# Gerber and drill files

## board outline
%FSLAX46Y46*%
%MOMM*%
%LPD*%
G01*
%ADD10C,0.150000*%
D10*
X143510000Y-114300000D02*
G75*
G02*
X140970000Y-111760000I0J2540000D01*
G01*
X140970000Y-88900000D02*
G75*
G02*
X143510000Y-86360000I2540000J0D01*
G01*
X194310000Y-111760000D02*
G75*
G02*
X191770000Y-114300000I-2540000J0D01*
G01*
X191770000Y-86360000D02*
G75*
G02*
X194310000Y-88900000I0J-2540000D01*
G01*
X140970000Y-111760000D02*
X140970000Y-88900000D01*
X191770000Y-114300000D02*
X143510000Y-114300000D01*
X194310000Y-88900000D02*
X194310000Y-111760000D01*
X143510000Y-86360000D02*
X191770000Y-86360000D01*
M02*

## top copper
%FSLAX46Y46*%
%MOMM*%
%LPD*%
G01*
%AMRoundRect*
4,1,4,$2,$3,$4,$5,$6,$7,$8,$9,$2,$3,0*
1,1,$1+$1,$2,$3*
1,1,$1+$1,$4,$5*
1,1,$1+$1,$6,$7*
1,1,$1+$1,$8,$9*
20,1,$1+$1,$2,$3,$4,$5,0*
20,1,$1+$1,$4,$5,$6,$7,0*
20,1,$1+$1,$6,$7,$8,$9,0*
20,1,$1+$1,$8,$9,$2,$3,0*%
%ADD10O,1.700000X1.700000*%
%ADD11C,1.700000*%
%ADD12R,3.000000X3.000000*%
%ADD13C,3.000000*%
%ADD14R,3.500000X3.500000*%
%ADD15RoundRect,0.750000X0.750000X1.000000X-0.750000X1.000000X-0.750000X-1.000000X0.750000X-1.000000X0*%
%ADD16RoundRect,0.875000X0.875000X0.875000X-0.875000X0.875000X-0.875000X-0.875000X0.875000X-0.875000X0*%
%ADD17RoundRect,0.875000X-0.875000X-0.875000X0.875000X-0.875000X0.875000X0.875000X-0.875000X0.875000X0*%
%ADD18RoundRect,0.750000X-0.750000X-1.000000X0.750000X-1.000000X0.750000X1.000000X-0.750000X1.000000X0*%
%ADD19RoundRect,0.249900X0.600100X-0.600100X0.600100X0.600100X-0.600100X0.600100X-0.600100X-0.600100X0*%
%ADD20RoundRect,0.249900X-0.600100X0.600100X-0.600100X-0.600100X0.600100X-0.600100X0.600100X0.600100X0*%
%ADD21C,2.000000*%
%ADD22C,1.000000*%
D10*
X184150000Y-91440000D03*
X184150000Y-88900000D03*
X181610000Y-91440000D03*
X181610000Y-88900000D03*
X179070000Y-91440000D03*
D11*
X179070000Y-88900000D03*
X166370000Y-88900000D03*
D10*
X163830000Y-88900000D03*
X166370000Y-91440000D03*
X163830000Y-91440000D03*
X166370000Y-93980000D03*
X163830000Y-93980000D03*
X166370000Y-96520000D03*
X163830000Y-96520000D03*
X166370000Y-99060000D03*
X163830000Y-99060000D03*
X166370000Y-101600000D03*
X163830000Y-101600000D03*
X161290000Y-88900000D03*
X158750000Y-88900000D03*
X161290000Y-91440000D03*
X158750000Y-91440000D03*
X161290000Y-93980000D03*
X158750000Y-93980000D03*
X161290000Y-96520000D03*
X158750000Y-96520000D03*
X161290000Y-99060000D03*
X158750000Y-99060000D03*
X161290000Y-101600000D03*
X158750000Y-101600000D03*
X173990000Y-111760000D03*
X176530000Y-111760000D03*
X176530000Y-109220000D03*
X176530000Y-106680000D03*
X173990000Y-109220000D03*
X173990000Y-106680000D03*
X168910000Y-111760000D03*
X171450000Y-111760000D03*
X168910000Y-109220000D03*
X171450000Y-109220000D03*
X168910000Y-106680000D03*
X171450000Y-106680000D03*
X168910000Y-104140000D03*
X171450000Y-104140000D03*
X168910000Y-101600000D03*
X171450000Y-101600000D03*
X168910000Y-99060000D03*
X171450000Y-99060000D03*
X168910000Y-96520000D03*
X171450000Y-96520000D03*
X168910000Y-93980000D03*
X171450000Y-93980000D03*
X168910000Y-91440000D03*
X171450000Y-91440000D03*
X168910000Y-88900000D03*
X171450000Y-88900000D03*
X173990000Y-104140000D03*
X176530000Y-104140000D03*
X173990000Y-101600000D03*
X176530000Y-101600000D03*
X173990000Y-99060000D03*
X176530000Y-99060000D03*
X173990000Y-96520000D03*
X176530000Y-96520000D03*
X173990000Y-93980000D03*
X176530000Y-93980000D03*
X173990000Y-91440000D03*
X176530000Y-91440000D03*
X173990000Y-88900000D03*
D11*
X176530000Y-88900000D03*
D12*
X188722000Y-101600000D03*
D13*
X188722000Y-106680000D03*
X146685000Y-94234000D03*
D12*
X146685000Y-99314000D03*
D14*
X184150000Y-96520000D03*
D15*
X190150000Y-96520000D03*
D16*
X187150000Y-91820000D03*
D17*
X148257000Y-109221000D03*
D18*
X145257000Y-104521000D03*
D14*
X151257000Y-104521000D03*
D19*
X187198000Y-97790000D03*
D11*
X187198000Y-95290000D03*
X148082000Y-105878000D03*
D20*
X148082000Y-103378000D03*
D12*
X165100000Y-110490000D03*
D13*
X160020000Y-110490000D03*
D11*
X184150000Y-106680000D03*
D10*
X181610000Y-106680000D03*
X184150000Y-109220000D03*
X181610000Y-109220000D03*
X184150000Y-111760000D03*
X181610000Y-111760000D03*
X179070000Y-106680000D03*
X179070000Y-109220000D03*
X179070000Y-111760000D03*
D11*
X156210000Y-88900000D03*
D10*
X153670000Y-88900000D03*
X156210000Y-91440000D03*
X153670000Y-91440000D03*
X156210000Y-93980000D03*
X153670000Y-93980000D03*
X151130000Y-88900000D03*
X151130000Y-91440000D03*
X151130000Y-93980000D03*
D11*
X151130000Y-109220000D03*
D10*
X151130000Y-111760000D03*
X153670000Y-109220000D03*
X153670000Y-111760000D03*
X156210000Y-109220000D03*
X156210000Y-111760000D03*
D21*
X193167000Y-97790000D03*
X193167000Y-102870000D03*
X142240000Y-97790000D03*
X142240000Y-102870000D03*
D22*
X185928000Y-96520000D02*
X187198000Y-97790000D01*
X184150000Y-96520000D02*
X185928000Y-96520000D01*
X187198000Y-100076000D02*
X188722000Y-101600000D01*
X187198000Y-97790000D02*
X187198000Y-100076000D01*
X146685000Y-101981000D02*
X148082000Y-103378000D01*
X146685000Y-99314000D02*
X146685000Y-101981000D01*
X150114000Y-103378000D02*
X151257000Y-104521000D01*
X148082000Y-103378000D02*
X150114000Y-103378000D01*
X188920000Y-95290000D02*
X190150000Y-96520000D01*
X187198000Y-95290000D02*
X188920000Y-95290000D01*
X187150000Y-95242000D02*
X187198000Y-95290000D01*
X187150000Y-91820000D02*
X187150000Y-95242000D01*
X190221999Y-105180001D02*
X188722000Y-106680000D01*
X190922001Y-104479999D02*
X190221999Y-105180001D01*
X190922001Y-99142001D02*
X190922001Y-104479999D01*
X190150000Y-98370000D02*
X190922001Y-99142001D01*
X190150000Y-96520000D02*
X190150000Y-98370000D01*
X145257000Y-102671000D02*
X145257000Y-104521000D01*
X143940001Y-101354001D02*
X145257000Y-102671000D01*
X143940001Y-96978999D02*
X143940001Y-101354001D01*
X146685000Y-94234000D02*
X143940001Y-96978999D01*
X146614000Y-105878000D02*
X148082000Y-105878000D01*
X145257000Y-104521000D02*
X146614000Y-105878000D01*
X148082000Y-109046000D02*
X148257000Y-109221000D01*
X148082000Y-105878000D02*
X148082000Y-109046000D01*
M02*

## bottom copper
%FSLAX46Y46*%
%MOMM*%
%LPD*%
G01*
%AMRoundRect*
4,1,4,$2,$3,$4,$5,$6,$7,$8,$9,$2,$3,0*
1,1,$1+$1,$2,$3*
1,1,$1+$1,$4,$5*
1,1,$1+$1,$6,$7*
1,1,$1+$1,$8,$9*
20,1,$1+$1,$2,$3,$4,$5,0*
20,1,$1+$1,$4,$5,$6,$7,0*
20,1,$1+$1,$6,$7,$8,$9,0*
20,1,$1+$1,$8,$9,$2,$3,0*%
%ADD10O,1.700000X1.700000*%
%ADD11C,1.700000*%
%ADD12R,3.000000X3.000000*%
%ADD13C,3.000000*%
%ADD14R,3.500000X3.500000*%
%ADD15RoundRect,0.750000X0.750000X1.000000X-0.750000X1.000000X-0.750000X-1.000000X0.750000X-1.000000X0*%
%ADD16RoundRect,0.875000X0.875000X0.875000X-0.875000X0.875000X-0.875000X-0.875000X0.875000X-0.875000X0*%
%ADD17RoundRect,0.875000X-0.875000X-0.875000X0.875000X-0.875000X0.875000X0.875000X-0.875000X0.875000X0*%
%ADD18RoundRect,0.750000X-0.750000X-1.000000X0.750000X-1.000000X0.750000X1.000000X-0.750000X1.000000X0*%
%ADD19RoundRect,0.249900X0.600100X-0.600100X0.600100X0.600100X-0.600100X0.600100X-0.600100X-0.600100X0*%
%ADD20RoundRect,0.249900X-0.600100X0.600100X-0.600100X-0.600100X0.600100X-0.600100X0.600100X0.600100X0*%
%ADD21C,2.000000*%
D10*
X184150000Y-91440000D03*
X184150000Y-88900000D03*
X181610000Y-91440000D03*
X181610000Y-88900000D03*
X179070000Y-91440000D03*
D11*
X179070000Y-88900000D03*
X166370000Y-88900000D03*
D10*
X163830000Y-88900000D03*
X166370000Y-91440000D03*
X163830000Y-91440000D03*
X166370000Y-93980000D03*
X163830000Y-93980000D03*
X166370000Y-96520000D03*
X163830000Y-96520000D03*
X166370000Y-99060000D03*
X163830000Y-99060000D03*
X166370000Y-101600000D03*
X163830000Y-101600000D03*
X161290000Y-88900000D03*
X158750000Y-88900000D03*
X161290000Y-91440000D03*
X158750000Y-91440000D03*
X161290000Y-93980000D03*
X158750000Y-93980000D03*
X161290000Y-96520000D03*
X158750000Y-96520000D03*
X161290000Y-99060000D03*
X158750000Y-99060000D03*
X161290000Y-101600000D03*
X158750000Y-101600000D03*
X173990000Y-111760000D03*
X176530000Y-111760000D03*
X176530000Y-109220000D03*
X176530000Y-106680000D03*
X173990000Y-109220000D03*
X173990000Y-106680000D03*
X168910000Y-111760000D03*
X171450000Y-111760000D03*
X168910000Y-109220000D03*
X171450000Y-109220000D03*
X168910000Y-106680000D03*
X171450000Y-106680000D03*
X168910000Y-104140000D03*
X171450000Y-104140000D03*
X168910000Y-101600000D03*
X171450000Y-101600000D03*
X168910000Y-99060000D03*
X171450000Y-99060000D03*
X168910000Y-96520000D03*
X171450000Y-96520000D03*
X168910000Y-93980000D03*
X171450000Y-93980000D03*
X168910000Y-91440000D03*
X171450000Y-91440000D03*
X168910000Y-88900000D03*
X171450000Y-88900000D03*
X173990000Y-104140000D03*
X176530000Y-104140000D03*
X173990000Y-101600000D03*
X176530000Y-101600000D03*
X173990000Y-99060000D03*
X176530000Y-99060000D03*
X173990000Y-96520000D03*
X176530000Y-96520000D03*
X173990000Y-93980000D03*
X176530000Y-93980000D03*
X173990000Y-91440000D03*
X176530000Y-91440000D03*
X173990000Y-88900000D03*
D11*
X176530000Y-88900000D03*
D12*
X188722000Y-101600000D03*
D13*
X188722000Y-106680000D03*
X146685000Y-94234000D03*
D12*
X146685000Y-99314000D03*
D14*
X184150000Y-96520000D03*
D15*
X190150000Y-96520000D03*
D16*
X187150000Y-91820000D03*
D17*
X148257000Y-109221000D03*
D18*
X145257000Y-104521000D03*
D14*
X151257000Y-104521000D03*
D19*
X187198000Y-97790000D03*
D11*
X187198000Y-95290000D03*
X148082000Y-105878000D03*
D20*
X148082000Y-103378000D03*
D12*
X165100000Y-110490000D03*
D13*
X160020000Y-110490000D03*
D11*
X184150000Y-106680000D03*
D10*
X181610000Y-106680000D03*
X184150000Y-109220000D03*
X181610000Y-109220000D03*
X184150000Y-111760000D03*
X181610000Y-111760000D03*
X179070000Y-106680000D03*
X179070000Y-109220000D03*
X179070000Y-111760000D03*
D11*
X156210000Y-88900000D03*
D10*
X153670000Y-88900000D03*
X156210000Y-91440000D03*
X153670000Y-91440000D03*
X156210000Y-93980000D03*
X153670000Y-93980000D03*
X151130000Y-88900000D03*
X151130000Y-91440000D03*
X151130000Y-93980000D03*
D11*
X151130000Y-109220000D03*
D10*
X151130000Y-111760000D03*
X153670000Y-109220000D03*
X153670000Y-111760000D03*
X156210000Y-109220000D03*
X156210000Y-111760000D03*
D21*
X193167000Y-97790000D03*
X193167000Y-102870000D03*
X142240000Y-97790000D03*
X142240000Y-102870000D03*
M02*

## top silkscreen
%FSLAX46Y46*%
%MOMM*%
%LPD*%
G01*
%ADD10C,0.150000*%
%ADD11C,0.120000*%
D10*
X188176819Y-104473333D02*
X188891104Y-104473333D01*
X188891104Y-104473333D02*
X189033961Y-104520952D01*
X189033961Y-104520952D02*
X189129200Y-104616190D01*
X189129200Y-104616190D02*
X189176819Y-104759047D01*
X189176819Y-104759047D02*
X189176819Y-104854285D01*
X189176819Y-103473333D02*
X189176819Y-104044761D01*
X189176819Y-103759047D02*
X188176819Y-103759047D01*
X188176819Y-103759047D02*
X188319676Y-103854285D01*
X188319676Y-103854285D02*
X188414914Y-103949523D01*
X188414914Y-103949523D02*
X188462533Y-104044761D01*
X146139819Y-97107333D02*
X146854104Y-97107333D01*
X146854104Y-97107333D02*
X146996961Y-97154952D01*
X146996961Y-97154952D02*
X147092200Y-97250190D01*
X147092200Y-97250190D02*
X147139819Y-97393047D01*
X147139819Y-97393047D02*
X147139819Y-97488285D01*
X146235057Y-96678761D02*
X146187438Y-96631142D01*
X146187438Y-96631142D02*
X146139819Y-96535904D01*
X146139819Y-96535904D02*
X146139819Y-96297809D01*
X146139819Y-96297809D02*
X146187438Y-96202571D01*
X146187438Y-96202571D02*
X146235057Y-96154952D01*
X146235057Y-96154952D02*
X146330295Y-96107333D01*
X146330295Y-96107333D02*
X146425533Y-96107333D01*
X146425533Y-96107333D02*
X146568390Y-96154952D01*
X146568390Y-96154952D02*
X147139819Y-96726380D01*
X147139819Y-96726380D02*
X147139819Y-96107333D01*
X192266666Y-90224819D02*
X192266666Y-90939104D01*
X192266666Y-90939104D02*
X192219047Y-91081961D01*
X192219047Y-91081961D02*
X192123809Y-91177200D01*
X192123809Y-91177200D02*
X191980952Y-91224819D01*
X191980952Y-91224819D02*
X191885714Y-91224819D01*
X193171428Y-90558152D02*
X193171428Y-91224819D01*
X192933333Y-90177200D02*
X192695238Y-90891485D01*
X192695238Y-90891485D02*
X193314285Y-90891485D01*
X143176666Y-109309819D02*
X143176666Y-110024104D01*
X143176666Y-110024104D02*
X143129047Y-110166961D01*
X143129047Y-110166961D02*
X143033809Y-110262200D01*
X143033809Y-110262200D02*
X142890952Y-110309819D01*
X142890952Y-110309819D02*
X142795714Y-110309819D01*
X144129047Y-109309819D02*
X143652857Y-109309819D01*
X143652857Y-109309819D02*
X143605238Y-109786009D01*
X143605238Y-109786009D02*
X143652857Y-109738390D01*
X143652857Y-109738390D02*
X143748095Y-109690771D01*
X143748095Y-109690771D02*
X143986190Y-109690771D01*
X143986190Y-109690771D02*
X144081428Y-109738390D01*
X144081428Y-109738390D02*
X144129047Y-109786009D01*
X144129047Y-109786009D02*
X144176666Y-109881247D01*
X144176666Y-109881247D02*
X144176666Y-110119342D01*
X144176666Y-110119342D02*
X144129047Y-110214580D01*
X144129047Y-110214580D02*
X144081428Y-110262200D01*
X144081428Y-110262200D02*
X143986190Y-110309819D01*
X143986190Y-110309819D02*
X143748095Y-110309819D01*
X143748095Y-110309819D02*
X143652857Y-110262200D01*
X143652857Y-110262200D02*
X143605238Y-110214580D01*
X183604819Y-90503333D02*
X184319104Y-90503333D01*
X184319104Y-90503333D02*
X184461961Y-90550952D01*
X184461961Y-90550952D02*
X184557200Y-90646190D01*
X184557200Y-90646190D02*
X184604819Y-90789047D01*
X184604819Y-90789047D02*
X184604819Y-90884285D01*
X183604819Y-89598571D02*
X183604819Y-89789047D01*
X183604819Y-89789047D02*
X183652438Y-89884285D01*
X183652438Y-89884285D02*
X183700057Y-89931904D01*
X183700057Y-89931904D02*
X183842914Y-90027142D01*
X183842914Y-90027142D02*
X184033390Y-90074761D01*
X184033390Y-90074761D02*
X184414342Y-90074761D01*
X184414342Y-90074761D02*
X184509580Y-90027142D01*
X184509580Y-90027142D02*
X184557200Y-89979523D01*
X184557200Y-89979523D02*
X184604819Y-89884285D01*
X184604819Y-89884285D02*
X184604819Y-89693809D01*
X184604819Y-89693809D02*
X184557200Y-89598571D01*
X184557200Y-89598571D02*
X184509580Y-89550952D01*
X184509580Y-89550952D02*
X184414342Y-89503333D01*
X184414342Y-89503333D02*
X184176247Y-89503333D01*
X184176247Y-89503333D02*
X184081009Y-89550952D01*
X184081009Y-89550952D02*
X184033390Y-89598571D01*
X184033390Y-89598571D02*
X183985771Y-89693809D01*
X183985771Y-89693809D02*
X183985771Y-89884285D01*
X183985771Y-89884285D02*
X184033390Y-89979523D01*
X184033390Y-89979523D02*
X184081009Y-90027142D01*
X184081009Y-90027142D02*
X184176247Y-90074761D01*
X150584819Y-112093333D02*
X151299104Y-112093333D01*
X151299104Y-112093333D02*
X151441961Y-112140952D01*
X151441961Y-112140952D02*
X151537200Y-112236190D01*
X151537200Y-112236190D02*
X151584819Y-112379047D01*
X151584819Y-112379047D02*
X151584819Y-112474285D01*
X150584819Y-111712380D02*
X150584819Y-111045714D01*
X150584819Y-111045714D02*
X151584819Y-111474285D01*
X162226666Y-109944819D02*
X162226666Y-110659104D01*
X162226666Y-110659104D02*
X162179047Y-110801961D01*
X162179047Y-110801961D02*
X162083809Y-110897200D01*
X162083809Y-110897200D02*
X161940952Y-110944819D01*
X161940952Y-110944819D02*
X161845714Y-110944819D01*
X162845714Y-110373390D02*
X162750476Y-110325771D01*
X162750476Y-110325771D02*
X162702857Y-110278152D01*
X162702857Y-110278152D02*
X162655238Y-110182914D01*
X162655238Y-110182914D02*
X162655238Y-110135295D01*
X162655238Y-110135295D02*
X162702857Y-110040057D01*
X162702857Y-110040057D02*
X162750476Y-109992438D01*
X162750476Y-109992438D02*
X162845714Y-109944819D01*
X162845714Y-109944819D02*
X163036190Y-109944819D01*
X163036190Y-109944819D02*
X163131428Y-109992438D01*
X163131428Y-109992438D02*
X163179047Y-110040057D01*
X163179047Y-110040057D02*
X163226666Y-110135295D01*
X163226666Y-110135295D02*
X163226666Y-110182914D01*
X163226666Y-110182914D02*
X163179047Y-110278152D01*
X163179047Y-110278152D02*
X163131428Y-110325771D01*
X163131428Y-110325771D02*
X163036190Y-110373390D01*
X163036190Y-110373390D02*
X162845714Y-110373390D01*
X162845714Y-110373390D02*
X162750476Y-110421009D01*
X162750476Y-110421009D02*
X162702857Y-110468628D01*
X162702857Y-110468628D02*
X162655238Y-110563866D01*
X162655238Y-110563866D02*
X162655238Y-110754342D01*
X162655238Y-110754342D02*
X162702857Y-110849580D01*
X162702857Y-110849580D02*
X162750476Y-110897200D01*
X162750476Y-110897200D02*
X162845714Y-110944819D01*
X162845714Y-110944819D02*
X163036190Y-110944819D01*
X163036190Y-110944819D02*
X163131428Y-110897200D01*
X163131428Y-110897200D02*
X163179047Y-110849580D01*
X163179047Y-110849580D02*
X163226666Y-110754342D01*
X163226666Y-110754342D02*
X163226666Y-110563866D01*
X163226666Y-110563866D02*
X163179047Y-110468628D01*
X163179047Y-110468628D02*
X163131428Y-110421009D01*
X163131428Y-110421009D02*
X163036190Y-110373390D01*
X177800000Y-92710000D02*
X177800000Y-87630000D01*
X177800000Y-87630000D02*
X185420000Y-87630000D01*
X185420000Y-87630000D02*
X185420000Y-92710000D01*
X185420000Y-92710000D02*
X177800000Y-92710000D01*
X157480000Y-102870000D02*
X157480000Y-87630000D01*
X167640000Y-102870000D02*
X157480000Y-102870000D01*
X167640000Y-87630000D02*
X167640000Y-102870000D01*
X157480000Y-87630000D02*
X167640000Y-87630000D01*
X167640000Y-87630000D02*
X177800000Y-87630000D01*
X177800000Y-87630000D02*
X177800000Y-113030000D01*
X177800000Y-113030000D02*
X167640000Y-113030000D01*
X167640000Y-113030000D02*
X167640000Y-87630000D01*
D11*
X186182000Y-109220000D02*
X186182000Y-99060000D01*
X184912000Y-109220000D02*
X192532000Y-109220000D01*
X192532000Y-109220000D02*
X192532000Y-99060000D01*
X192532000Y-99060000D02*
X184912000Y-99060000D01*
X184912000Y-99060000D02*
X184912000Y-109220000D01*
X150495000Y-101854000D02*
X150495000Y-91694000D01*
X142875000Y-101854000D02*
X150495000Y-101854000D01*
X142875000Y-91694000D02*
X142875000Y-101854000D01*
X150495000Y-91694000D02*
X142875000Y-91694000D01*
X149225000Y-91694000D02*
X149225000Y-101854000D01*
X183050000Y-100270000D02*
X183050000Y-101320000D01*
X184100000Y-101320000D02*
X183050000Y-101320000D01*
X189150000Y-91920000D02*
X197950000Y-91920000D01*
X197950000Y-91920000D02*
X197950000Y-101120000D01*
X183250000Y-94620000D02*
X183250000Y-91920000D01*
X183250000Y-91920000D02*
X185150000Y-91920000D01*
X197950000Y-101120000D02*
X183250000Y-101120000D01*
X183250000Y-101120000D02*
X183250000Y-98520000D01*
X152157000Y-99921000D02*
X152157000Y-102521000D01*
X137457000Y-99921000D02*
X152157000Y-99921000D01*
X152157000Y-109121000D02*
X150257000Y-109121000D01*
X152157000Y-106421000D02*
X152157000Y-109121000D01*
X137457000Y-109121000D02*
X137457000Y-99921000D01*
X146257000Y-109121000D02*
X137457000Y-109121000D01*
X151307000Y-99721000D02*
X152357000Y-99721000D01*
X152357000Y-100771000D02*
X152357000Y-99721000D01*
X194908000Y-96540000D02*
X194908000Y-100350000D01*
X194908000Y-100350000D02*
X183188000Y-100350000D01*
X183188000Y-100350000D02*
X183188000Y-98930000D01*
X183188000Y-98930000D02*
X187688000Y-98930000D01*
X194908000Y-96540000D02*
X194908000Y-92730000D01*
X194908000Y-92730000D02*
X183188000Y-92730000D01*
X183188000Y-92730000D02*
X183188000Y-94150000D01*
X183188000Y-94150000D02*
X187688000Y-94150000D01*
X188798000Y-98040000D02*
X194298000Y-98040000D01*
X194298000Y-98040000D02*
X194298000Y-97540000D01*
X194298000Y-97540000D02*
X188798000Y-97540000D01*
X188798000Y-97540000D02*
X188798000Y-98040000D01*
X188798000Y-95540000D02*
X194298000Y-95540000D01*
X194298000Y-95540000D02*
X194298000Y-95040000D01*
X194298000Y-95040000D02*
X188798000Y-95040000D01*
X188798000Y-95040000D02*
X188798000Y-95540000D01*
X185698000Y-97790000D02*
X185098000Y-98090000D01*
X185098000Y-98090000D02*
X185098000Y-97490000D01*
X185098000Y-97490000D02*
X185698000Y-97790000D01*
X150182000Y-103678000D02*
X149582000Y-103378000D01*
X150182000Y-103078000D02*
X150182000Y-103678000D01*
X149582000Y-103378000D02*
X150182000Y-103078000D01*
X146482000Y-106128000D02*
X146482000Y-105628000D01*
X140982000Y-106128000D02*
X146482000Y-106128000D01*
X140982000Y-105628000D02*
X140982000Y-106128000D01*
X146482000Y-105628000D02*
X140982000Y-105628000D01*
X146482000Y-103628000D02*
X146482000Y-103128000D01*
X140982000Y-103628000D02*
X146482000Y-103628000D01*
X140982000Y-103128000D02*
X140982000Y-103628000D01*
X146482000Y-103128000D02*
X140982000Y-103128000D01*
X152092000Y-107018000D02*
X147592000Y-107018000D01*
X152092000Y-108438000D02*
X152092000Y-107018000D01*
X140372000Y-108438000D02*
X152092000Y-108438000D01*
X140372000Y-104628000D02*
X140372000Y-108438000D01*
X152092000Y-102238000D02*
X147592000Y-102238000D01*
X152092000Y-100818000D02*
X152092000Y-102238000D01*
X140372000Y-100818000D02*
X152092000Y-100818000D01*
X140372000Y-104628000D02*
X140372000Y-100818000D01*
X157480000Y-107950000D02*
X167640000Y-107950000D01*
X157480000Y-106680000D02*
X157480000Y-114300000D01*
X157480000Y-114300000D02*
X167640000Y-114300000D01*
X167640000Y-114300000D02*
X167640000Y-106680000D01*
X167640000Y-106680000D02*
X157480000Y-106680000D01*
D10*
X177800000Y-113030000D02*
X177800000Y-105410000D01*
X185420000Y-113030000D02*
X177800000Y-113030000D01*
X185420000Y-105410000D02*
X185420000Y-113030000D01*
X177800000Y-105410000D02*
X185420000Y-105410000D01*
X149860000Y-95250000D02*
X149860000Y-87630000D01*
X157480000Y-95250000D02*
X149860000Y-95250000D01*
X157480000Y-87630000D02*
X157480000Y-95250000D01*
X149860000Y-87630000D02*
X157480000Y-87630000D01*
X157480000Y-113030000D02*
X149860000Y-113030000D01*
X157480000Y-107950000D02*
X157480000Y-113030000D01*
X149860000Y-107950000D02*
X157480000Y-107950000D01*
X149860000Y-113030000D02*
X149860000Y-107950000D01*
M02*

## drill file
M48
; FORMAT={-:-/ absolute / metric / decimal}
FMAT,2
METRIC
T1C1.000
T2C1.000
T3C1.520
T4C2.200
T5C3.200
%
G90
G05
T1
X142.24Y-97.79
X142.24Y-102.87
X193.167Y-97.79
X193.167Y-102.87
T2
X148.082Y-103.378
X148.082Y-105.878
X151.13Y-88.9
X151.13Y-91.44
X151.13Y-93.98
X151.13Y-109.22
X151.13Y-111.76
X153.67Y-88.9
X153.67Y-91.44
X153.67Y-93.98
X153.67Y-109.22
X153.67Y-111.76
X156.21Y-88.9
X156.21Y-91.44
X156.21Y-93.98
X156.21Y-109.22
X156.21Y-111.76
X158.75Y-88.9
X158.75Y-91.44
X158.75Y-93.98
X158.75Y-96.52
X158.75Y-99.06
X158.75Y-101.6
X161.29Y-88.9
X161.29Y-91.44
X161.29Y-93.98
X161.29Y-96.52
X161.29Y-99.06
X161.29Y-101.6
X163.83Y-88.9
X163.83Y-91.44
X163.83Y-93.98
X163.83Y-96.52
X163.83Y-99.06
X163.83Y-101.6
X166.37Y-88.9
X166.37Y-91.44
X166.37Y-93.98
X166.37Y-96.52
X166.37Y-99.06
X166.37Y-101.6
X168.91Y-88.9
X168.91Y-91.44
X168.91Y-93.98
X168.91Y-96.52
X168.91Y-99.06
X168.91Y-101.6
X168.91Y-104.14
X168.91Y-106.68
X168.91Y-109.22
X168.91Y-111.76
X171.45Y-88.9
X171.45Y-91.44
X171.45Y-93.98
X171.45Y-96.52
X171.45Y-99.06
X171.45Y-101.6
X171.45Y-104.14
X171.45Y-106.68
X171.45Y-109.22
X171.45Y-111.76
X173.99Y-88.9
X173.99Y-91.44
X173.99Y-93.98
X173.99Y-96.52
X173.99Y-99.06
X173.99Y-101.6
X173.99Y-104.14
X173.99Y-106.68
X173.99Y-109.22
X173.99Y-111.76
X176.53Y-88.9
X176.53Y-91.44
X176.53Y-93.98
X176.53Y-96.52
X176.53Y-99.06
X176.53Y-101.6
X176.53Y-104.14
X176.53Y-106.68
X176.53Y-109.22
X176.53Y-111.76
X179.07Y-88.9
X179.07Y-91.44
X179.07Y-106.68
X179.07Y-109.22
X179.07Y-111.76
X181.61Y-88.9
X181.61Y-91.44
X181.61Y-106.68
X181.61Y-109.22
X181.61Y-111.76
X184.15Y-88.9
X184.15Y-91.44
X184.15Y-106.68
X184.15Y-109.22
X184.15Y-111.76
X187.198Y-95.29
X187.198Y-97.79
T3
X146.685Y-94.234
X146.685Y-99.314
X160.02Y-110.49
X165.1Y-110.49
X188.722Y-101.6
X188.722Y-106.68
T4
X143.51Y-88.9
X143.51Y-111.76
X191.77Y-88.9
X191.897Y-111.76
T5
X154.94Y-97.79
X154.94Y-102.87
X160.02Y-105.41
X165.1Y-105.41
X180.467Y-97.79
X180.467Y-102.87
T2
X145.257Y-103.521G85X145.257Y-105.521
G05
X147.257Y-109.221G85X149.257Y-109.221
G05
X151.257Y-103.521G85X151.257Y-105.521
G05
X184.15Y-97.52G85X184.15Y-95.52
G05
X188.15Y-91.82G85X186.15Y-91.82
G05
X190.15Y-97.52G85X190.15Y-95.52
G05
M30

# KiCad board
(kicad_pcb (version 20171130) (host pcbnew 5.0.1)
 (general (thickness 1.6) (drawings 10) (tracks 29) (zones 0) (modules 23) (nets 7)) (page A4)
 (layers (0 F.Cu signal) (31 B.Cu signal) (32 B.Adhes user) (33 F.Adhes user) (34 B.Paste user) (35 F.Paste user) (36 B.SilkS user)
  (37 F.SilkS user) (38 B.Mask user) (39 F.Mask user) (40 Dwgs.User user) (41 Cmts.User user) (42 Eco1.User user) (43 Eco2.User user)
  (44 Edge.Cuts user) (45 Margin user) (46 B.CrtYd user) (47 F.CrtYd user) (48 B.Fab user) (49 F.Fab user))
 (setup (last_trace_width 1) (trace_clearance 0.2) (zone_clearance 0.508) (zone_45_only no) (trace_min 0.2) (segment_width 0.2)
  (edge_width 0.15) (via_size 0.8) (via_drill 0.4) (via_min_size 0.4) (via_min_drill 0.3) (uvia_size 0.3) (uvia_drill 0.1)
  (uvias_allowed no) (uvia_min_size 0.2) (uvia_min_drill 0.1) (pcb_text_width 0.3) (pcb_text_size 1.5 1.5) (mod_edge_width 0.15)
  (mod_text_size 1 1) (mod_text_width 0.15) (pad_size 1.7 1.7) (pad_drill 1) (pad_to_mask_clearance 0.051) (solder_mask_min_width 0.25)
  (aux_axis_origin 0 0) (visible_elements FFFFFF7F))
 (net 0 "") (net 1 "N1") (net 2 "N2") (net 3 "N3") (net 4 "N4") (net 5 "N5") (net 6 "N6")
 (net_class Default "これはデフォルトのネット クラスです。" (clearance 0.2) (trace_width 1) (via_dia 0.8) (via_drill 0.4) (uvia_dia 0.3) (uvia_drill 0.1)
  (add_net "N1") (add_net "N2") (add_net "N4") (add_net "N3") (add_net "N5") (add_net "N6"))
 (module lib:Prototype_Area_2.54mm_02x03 (layer F.Cu) (at 179.07 88.9 90)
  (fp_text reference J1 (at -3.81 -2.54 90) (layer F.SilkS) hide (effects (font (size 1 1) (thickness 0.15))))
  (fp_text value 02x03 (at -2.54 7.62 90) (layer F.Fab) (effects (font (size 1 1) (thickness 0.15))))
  (fp_line (start -3.81 -1.27) (end 1.27 -1.27) (layer F.SilkS) (width 0.15))
  (fp_line (start 1.27 -1.27) (end 1.27 6.35) (layer F.SilkS) (width 0.15))
  (fp_line (start 1.27 6.35) (end -3.81 6.35) (layer F.SilkS) (width 0.15))
  (fp_line (start -3.81 6.35) (end -3.81 -1.27) (layer F.SilkS) (width 0.15))
  (pad 6 thru_hole oval (at -2.54 5.08 90) (size 1.7 1.7) (drill 1) (layers *.Cu *.Mask))
  (pad 5 thru_hole oval (at 0 5.08 90) (size 1.7 1.7) (drill 1) (layers *.Cu *.Mask))
  (pad 4 thru_hole oval (at -2.54 2.54 90) (size 1.7 1.7) (drill 1) (layers *.Cu *.Mask))
  (pad 3 thru_hole oval (at 0 2.54 90) (size 1.7 1.7) (drill 1) (layers *.Cu *.Mask))
  (pad 2 thru_hole oval (at -2.54 0 90) (size 1.7 1.7) (drill 1) (layers *.Cu *.Mask))
  (pad 1 thru_hole circle (at 0 0 90) (size 1.7 1.7) (drill 1) (layers *.Cu *.Mask)))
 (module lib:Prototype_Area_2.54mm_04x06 (layer F.Cu) (at 166.37 88.9)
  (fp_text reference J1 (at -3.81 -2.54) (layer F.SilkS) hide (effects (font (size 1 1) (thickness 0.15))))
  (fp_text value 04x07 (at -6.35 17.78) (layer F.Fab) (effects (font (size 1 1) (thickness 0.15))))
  (fp_line (start -8.89 13.97) (end -8.89 -1.27) (layer F.SilkS) (width 0.15))
  (fp_line (start 1.27 13.97) (end -8.89 13.97) (layer F.SilkS) (width 0.15))
  (fp_line (start 1.27 -1.27) (end 1.27 13.97) (layer F.SilkS) (width 0.15))
  (fp_line (start -8.89 -1.27) (end 1.27 -1.27) (layer F.SilkS) (width 0.15))
  (pad 1 thru_hole circle (at 0 0) (size 1.7 1.7) (drill 1) (layers *.Cu *.Mask))
  (pad 2 thru_hole oval (at -2.54 0) (size 1.7 1.7) (drill 1) (layers *.Cu *.Mask))
  (pad 7 thru_hole oval (at 0 2.54) (size 1.7 1.7) (drill 1) (layers *.Cu *.Mask))
  (pad 8 thru_hole oval (at -2.54 2.54) (size 1.7 1.7) (drill 1) (layers *.Cu *.Mask))
  (pad 13 thru_hole oval (at 0 5.08) (size 1.7 1.7) (drill 1) (layers *.Cu *.Mask))
  (pad 14 thru_hole oval (at -2.54 5.08) (size 1.7 1.7) (drill 1) (layers *.Cu *.Mask))
  (pad 19 thru_hole oval (at 0 7.62) (size 1.7 1.7) (drill 1) (layers *.Cu *.Mask))
  (pad 20 thru_hole oval (at -2.54 7.62) (size 1.7 1.7) (drill 1) (layers *.Cu *.Mask))
  (pad 25 thru_hole oval (at 0 10.16) (size 1.7 1.7) (drill 1) (layers *.Cu *.Mask))
  (pad 26 thru_hole oval (at -2.54 10.16) (size 1.7 1.7) (drill 1) (layers *.Cu *.Mask))
  (pad 31 thru_hole oval (at 0 12.7) (size 1.7 1.7) (drill 1) (layers *.Cu *.Mask))
  (pad 32 thru_hole oval (at -2.54 12.7) (size 1.7 1.7) (drill 1) (layers *.Cu *.Mask))
  (pad 3 thru_hole oval (at -5.08 0) (size 1.7 1.7) (drill 1) (layers *.Cu *.Mask))
  (pad 4 thru_hole oval (at -7.62 0) (size 1.7 1.7) (drill 1) (layers *.Cu *.Mask))
  (pad 9 thru_hole oval (at -5.08 2.54) (size 1.7 1.7) (drill 1) (layers *.Cu *.Mask))
  (pad 10 thru_hole oval (at -7.62 2.54) (size 1.7 1.7) (drill 1) (layers *.Cu *.Mask))
  (pad 15 thru_hole oval (at -5.08 5.08) (size 1.7 1.7) (drill 1) (layers *.Cu *.Mask))
  (pad 16 thru_hole oval (at -7.62 5.08) (size 1.7 1.7) (drill 1) (layers *.Cu *.Mask))
  (pad 21 thru_hole oval (at -5.08 7.62) (size 1.7 1.7) (drill 1) (layers *.Cu *.Mask))
  (pad 22 thru_hole oval (at -7.62 7.62) (size 1.7 1.7) (drill 1) (layers *.Cu *.Mask))
  (pad 27 thru_hole oval (at -5.08 10.16) (size 1.7 1.7) (drill 1) (layers *.Cu *.Mask))
  (pad 28 thru_hole oval (at -7.62 10.16) (size 1.7 1.7) (drill 1) (layers *.Cu *.Mask))
  (pad 33 thru_hole oval (at -5.08 12.7) (size 1.7 1.7) (drill 1) (layers *.Cu *.Mask))
  (pad 34 thru_hole oval (at -7.62 12.7) (size 1.7 1.7) (drill 1) (layers *.Cu *.Mask)))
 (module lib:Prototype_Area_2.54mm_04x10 (layer F.Cu) (at 176.53 88.9)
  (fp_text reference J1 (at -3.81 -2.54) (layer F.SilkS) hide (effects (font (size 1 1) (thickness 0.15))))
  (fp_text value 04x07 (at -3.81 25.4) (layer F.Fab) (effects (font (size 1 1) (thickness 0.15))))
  (fp_line (start -8.89 -1.27) (end 1.27 -1.27) (layer F.SilkS) (width 0.15))
  (fp_line (start 1.27 -1.27) (end 1.27 24.13) (layer F.SilkS) (width 0.15))
  (fp_line (start 1.27 24.13) (end -8.89 24.13) (layer F.SilkS) (width 0.15))
  (fp_line (start -8.89 24.13) (end -8.89 -1.27) (layer F.SilkS) (width 0.15))
  (pad 38 thru_hole oval (at -2.54 22.86) (size 1.7 1.7) (drill 1) (layers *.Cu *.Mask))
  (pad 37 thru_hole oval (at 0 22.86) (size 1.7 1.7) (drill 1) (layers *.Cu *.Mask))
  (pad 33 thru_hole oval (at 0 20.32) (size 1.7 1.7) (drill 1) (layers *.Cu *.Mask))
  (pad 29 thru_hole oval (at 0 17.78) (size 1.7 1.7) (drill 1) (layers *.Cu *.Mask))
  (pad 34 thru_hole oval (at -2.54 20.32) (size 1.7 1.7) (drill 1) (layers *.Cu *.Mask))
  (pad 30 thru_hole oval (at -2.54 17.78) (size 1.7 1.7) (drill 1) (layers *.Cu *.Mask))
  (pad 40 thru_hole oval (at -7.62 22.86) (size 1.7 1.7) (drill 1) (layers *.Cu *.Mask))
  (pad 39 thru_hole oval (at -5.08 22.86) (size 1.7 1.7) (drill 1) (layers *.Cu *.Mask))
  (pad 36 thru_hole oval (at -7.62 20.32) (size 1.7 1.7) (drill 1) (layers *.Cu *.Mask))
  (pad 35 thru_hole oval (at -5.08 20.32) (size 1.7 1.7) (drill 1) (layers *.Cu *.Mask))
  (pad 32 thru_hole oval (at -7.62 17.78) (size 1.7 1.7) (drill 1) (layers *.Cu *.Mask))
  (pad 31 thru_hole oval (at -5.08 17.78) (size 1.7 1.7) (drill 1) (layers *.Cu *.Mask))
  (pad 28 thru_hole oval (at -7.62 15.24) (size 1.7 1.7) (drill 1) (layers *.Cu *.Mask))
  (pad 27 thru_hole oval (at -5.08 15.24) (size 1.7 1.7) (drill 1) (layers *.Cu *.Mask))
  (pad 24 thru_hole oval (at -7.62 12.7) (size 1.7 1.7) (drill 1) (layers *.Cu *.Mask))
  (pad 23 thru_hole oval (at -5.08 12.7) (size 1.7 1.7) (drill 1) (layers *.Cu *.Mask))
  (pad 20 thru_hole oval (at -7.62 10.16) (size 1.7 1.7) (drill 1) (layers *.Cu *.Mask))
  (pad 19 thru_hole oval (at -5.08 10.16) (size 1.7 1.7) (drill 1) (layers *.Cu *.Mask))
  (pad 16 thru_hole oval (at -7.62 7.62) (size 1.7 1.7) (drill 1) (layers *.Cu *.Mask))
  (pad 15 thru_hole oval (at -5.08 7.62) (size 1.7 1.7) (drill 1) (layers *.Cu *.Mask))
  (pad 12 thru_hole oval (at -7.62 5.08) (size 1.7 1.7) (drill 1) (layers *.Cu *.Mask))
  (pad 11 thru_hole oval (at -5.08 5.08) (size 1.7 1.7) (drill 1) (layers *.Cu *.Mask))
  (pad 8 thru_hole oval (at -7.62 2.54) (size 1.7 1.7) (drill 1) (layers *.Cu *.Mask))
  (pad 7 thru_hole oval (at -5.08 2.54) (size 1.7 1.7) (drill 1) (layers *.Cu *.Mask))
  (pad 4 thru_hole oval (at -7.62 0) (size 1.7 1.7) (drill 1) (layers *.Cu *.Mask))
  (pad 3 thru_hole oval (at -5.08 0) (size 1.7 1.7) (drill 1) (layers *.Cu *.Mask))
  (pad 26 thru_hole oval (at -2.54 15.24) (size 1.7 1.7) (drill 1) (layers *.Cu *.Mask))
  (pad 25 thru_hole oval (at 0 15.24) (size 1.7 1.7) (drill 1) (layers *.Cu *.Mask))
  (pad 22 thru_hole oval (at -2.54 12.7) (size 1.7 1.7) (drill 1) (layers *.Cu *.Mask))
  (pad 21 thru_hole oval (at 0 12.7) (size 1.7 1.7) (drill 1) (layers *.Cu *.Mask))
  (pad 18 thru_hole oval (at -2.54 10.16) (size 1.7 1.7) (drill 1) (layers *.Cu *.Mask))
  (pad 17 thru_hole oval (at 0 10.16) (size 1.7 1.7) (drill 1) (layers *.Cu *.Mask))
  (pad 14 thru_hole oval (at -2.54 7.62) (size 1.7 1.7) (drill 1) (layers *.Cu *.Mask))
  (pad 13 thru_hole oval (at 0 7.62) (size 1.7 1.7) (drill 1) (layers *.Cu *.Mask))
  (pad 10 thru_hole oval (at -2.54 5.08) (size 1.7 1.7) (drill 1) (layers *.Cu *.Mask))
  (pad 9 thru_hole oval (at 0 5.08) (size 1.7 1.7) (drill 1) (layers *.Cu *.Mask))
  (pad 6 thru_hole oval (at -2.54 2.54) (size 1.7 1.7) (drill 1) (layers *.Cu *.Mask))
  (pad 5 thru_hole oval (at 0 2.54) (size 1.7 1.7) (drill 1) (layers *.Cu *.Mask))
  (pad 2 thru_hole oval (at -2.54 0) (size 1.7 1.7) (drill 1) (layers *.Cu *.Mask))
  (pad 1 thru_hole circle (at 0 0) (size 1.7 1.7) (drill 1) (layers *.Cu *.Mask)))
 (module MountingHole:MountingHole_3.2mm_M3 (layer F.Cu) (at 160.02 105.41)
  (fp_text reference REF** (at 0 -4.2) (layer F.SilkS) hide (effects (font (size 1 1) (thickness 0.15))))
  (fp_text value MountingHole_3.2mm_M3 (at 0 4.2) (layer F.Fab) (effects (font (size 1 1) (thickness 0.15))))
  (pad 1 np_thru_hole circle (at 0 0) (size 3.2 3.2) (drill 3.2) (layers *.Cu *.Mask)))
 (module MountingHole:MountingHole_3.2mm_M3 (layer F.Cu) (at 165.1 105.41)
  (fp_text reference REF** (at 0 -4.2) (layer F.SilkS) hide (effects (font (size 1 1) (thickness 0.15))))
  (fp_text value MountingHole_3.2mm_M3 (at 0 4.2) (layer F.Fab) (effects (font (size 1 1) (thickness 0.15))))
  (pad 1 np_thru_hole circle (at 0 0) (size 3.2 3.2) (drill 3.2) (layers *.Cu *.Mask)))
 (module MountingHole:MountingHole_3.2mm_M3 (layer F.Cu) (at 180.467 102.87)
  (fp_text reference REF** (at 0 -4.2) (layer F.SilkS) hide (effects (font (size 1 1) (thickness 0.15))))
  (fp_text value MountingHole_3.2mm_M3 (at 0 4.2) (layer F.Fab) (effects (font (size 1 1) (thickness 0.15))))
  (pad 1 np_thru_hole circle (at 0 0) (size 3.2 3.2) (drill 3.2) (layers *.Cu *.Mask)))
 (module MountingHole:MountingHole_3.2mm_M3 (layer F.Cu) (at 180.467 97.79)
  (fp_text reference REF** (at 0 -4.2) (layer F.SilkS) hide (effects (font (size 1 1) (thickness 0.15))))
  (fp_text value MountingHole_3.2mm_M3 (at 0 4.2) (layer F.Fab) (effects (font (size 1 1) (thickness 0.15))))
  (pad 1 np_thru_hole circle (at 0 0) (size 3.2 3.2) (drill 3.2) (layers *.Cu *.Mask)))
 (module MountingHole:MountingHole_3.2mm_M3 (layer F.Cu) (at 154.94 102.87)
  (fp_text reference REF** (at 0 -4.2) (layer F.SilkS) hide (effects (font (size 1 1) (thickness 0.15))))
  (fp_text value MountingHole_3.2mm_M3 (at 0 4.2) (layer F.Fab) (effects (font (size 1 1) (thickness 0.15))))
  (pad 1 np_thru_hole circle (at 0 0) (size 3.2 3.2) (drill 3.2) (layers *.Cu *.Mask)))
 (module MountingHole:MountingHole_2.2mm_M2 (layer F.Cu) (at 191.77 88.9)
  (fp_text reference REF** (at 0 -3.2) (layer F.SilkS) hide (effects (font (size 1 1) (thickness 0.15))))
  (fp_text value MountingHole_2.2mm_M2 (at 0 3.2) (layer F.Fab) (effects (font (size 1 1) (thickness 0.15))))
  (pad 1 np_thru_hole circle (at 0 0) (size 2.2 2.2) (drill 2.2) (layers *.Cu *.Mask)))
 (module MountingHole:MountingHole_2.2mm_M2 (layer F.Cu) (at 191.897 111.76)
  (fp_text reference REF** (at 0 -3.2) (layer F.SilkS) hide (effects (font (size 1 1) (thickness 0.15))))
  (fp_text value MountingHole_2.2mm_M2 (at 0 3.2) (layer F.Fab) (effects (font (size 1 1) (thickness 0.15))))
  (pad 1 np_thru_hole circle (at 0 0) (size 2.2 2.2) (drill 2.2) (layers *.Cu *.Mask)))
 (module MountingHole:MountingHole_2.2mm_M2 (layer F.Cu) (at 143.51 88.9)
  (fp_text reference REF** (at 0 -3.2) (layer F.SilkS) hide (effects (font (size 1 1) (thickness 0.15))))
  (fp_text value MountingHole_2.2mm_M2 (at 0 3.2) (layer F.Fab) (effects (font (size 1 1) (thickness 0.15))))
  (pad 1 np_thru_hole circle (at 0 0) (size 2.2 2.2) (drill 2.2) (layers *.Cu *.Mask)))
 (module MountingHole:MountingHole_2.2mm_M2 (layer F.Cu) (at 143.51 111.76)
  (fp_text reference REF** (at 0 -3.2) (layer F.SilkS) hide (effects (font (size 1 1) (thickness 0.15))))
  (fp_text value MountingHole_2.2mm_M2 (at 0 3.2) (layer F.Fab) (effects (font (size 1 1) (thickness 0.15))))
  (pad 1 np_thru_hole circle (at 0 0) (size 2.2 2.2) (drill 2.2) (layers *.Cu *.Mask)))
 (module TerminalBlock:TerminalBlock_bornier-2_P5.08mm (layer F.Cu) (at 188.722 101.6 270)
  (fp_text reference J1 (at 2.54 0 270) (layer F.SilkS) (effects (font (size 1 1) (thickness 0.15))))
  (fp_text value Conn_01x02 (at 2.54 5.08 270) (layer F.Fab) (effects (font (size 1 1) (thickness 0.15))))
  (fp_line (start 7.62 2.54) (end -2.54 2.54) (layer F.SilkS) (width 0.12))
  (fp_line (start 7.62 3.81) (end 7.62 -3.81) (layer F.SilkS) (width 0.12))
  (fp_line (start 7.62 -3.81) (end -2.54 -3.81) (layer F.SilkS) (width 0.12))
  (fp_line (start -2.54 -3.81) (end -2.54 3.81) (layer F.SilkS) (width 0.12))
  (fp_line (start -2.54 3.81) (end 7.62 3.81) (layer F.SilkS) (width 0.12))
  (pad 1 thru_hole rect (at 0 0 270) (size 3 3) (drill 1.52) (layers *.Cu *.Mask) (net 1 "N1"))
  (pad 2 thru_hole circle (at 5.08 0 270) (size 3 3) (drill 1.52) (layers *.Cu *.Mask) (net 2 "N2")))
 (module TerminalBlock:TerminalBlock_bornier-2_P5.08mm (layer F.Cu) (at 146.685 99.314 90)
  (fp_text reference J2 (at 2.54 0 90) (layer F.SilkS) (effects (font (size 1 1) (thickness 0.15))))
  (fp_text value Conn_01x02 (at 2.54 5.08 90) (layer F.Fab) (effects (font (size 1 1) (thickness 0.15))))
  (fp_line (start -2.54 3.81) (end 7.62 3.81) (layer F.SilkS) (width 0.12))
  (fp_line (start -2.54 -3.81) (end -2.54 3.81) (layer F.SilkS) (width 0.12))
  (fp_line (start 7.62 -3.81) (end -2.54 -3.81) (layer F.SilkS) (width 0.12))
  (fp_line (start 7.62 3.81) (end 7.62 -3.81) (layer F.SilkS) (width 0.12))
  (fp_line (start 7.62 2.54) (end -2.54 2.54) (layer F.SilkS) (width 0.12))
  (pad 2 thru_hole circle (at 5.08 0 90) (size 3 3) (drill 1.52) (layers *.Cu *.Mask) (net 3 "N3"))
  (pad 1 thru_hole rect (at 0 0 90) (size 3 3) (drill 1.52) (layers *.Cu *.Mask) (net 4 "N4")))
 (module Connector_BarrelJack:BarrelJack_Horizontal (layer F.Cu) (at 184.15 96.52 180)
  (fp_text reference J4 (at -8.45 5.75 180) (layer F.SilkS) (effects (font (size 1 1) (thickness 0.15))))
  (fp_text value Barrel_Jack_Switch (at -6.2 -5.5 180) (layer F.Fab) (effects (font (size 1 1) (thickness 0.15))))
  (fp_line (start 1.1 -3.75) (end 1.1 -4.8) (layer F.SilkS) (width 0.12))
  (fp_line (start 0.05 -4.8) (end 1.1 -4.8) (layer F.SilkS) (width 0.12))
  (fp_line (start -5 4.6) (end -13.8 4.6) (layer F.SilkS) (width 0.12))
  (fp_line (start -13.8 4.6) (end -13.8 -4.6) (layer F.SilkS) (width 0.12))
  (fp_line (start 0.9 1.9) (end 0.9 4.6) (layer F.SilkS) (width 0.12))
  (fp_line (start 0.9 4.6) (end -1 4.6) (layer F.SilkS) (width 0.12))
  (fp_line (start -13.8 -4.6) (end 0.9 -4.6) (layer F.SilkS) (width 0.12))
  (fp_line (start 0.9 -4.6) (end 0.9 -2) (layer F.SilkS) (width 0.12))
  (pad 1 thru_hole rect (at 0 0 180) (size 3.5 3.5) (drill oval 1 3) (layers *.Cu *.Mask) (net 1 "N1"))
  (pad 2 thru_hole roundrect (at -6 0 180) (size 3 3.5) (drill oval 1 3) (layers *.Cu *.Mask) (roundrect_rratio 0.25) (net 2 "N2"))
  (pad 3 thru_hole roundrect (at -3 4.7 180) (size 3.5 3.5) (drill oval 3 1) (layers *.Cu *.Mask) (roundrect_rratio 0.25) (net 2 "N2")))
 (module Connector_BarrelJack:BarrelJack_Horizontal (layer F.Cu) (at 151.257 104.521)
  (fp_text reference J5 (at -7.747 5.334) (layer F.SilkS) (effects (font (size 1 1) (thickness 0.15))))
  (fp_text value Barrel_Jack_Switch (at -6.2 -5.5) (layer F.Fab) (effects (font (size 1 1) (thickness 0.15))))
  (fp_line (start 0.9 -4.6) (end 0.9 -2) (layer F.SilkS) (width 0.12))
  (fp_line (start -13.8 -4.6) (end 0.9 -4.6) (layer F.SilkS) (width 0.12))
  (fp_line (start 0.9 4.6) (end -1 4.6) (layer F.SilkS) (width 0.12))
  (fp_line (start 0.9 1.9) (end 0.9 4.6) (layer F.SilkS) (width 0.12))
  (fp_line (start -13.8 4.6) (end -13.8 -4.6) (layer F.SilkS) (width 0.12))
  (fp_line (start -5 4.6) (end -13.8 4.6) (layer F.SilkS) (width 0.12))
  (fp_line (start 0.05 -4.8) (end 1.1 -4.8) (layer F.SilkS) (width 0.12))
  (fp_line (start 1.1 -3.75) (end 1.1 -4.8) (layer F.SilkS) (width 0.12))
  (pad 3 thru_hole roundrect (at -3 4.7) (size 3.5 3.5) (drill oval 3 1) (layers *.Cu *.Mask) (roundrect_rratio 0.25) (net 3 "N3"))
  (pad 2 thru_hole roundrect (at -6 0) (size 3 3.5) (drill oval 1 3) (layers *.Cu *.Mask) (roundrect_rratio 0.25) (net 3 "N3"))
  (pad 1 thru_hole rect (at 0 0) (size 3.5 3.5) (drill oval 1 3) (layers *.Cu *.Mask) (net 4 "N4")))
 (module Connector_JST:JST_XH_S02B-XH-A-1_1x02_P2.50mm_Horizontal (layer F.Cu) (at 187.198 97.79 90)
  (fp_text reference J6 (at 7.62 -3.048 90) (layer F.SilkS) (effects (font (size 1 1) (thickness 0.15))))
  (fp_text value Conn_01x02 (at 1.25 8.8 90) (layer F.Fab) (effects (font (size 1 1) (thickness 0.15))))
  (fp_line (start 1.25 7.71) (end -2.56 7.71) (layer F.SilkS) (width 0.12))
  (fp_line (start -2.56 7.71) (end -2.56 -4.01) (layer F.SilkS) (width 0.12))
  (fp_line (start -2.56 -4.01) (end -1.14 -4.01) (layer F.SilkS) (width 0.12))
  (fp_line (start -1.14 -4.01) (end -1.14 0.49) (layer F.SilkS) (width 0.12))
  (fp_line (start 1.25 7.71) (end 5.06 7.71) (layer F.SilkS) (width 0.12))
  (fp_line (start 5.06 7.71) (end 5.06 -4.01) (layer F.SilkS) (width 0.12))
  (fp_line (start 5.06 -4.01) (end 3.64 -4.01) (layer F.SilkS) (width 0.12))
  (fp_line (start 3.64 -4.01) (end 3.64 0.49) (layer F.SilkS) (width 0.12))
  (fp_line (start -0.25 1.6) (end -0.25 7.1) (layer F.SilkS) (width 0.12))
  (fp_line (start -0.25 7.1) (end 0.25 7.1) (layer F.SilkS) (width 0.12))
  (fp_line (start 0.25 7.1) (end 0.25 1.6) (layer F.SilkS) (width 0.12))
  (fp_line (start 0.25 1.6) (end -0.25 1.6) (layer F.SilkS) (width 0.12))
  (fp_line (start 2.25 1.6) (end 2.25 7.1) (layer F.SilkS) (width 0.12))
  (fp_line (start 2.25 7.1) (end 2.75 7.1) (layer F.SilkS) (width 0.12))
  (fp_line (start 2.75 7.1) (end 2.75 1.6) (layer F.SilkS) (width 0.12))
  (fp_line (start 2.75 1.6) (end 2.25 1.6) (layer F.SilkS) (width 0.12))
  (fp_line (start 0 -1.5) (end -0.3 -2.1) (layer F.SilkS) (width 0.12))
  (fp_line (start -0.3 -2.1) (end 0.3 -2.1) (layer F.SilkS) (width 0.12))
  (fp_line (start 0.3 -2.1) (end 0 -1.5) (layer F.SilkS) (width 0.12))
  (pad 1 thru_hole roundrect (at 0 0 90) (size 1.7 1.7) (drill 1) (layers *.Cu *.Mask) (roundrect_rratio 0.147) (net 1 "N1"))
  (pad 2 thru_hole circle (at 2.5 0 90) (size 1.7 1.7) (drill 1) (layers *.Cu *.Mask) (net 2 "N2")))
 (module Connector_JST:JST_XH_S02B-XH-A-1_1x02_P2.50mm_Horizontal (layer F.Cu) (at 148.082 103.378 270)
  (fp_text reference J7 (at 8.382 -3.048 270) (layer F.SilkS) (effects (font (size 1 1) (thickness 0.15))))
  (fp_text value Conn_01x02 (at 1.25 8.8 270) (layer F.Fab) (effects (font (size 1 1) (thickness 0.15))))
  (fp_line (start 0.3 -2.1) (end 0 -1.5) (layer F.SilkS) (width 0.12))
  (fp_line (start -0.3 -2.1) (end 0.3 -2.1) (layer F.SilkS) (width 0.12))
  (fp_line (start 0 -1.5) (end -0.3 -2.1) (layer F.SilkS) (width 0.12))
  (fp_line (start 2.75 1.6) (end 2.25 1.6) (layer F.SilkS) (width 0.12))
  (fp_line (start 2.75 7.1) (end 2.75 1.6) (layer F.SilkS) (width 0.12))
  (fp_line (start 2.25 7.1) (end 2.75 7.1) (layer F.SilkS) (width 0.12))
  (fp_line (start 2.25 1.6) (end 2.25 7.1) (layer F.SilkS) (width 0.12))
  (fp_line (start 0.25 1.6) (end -0.25 1.6) (layer F.SilkS) (width 0.12))
  (fp_line (start 0.25 7.1) (end 0.25 1.6) (layer F.SilkS) (width 0.12))
  (fp_line (start -0.25 7.1) (end 0.25 7.1) (layer F.SilkS) (width 0.12))
  (fp_line (start -0.25 1.6) (end -0.25 7.1) (layer F.SilkS) (width 0.12))
  (fp_line (start 3.64 -4.01) (end 3.64 0.49) (layer F.SilkS) (width 0.12))
  (fp_line (start 5.06 -4.01) (end 3.64 -4.01) (layer F.SilkS) (width 0.12))
  (fp_line (start 5.06 7.71) (end 5.06 -4.01) (layer F.SilkS) (width 0.12))
  (fp_line (start 1.25 7.71) (end 5.06 7.71) (layer F.SilkS) (width 0.12))
  (fp_line (start -1.14 -4.01) (end -1.14 0.49) (layer F.SilkS) (width 0.12))
  (fp_line (start -2.56 -4.01) (end -1.14 -4.01) (layer F.SilkS) (width 0.12))
  (fp_line (start -2.56 7.71) (end -2.56 -4.01) (layer F.SilkS) (width 0.12))
  (fp_line (start 1.25 7.71) (end -2.56 7.71) (layer F.SilkS) (width 0.12))
  (pad 2 thru_hole circle (at 2.5 0 270) (size 1.7 1.7) (drill 1) (layers *.Cu *.Mask) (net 3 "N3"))
  (pad 1 thru_hole roundrect (at 0 0 270) (size 1.7 1.7) (drill 1) (layers *.Cu *.Mask) (roundrect_rratio 0.147) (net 4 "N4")))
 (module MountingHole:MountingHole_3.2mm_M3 (layer F.Cu) (at 154.94 97.79)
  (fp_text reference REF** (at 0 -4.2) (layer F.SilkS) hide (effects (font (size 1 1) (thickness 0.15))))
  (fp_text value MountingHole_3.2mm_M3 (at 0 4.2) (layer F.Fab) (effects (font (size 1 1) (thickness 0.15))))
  (pad 1 np_thru_hole circle (at 0 0) (size 3.2 3.2) (drill 3.2) (layers *.Cu *.Mask)))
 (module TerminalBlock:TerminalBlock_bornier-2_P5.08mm (layer F.Cu) (at 165.1 110.49 180)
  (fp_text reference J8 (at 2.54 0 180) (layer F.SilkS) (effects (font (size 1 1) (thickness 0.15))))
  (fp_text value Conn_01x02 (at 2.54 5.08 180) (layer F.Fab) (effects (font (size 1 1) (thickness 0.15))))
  (fp_line (start 7.62 2.54) (end -2.54 2.54) (layer F.SilkS) (width 0.12))
  (fp_line (start 7.62 3.81) (end 7.62 -3.81) (layer F.SilkS) (width 0.12))
  (fp_line (start 7.62 -3.81) (end -2.54 -3.81) (layer F.SilkS) (width 0.12))
  (fp_line (start -2.54 -3.81) (end -2.54 3.81) (layer F.SilkS) (width 0.12))
  (fp_line (start -2.54 3.81) (end 7.62 3.81) (layer F.SilkS) (width 0.12))
  (pad 1 thru_hole rect (at 0 0 180) (size 3 3) (drill 1.52) (layers *.Cu *.Mask) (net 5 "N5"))
  (pad 2 thru_hole circle (at 5.08 0 180) (size 3 3) (drill 1.52) (layers *.Cu *.Mask) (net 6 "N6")))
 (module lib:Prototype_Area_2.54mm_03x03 (layer F.Cu) (at 184.15 106.68)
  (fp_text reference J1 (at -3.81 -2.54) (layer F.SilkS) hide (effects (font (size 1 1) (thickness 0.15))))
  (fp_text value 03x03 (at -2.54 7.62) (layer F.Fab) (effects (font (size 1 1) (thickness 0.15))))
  (fp_line (start -6.35 6.35) (end -6.35 -1.27) (layer F.SilkS) (width 0.15))
  (fp_line (start 1.27 6.35) (end -6.35 6.35) (layer F.SilkS) (width 0.15))
  (fp_line (start 1.27 -1.27) (end 1.27 6.35) (layer F.SilkS) (width 0.15))
  (fp_line (start -6.35 -1.27) (end 1.27 -1.27) (layer F.SilkS) (width 0.15))
  (pad 1 thru_hole circle (at 0 0) (size 1.7 1.7) (drill 1) (layers *.Cu *.Mask))
  (pad 2 thru_hole oval (at -2.54 0) (size 1.7 1.7) (drill 1) (layers *.Cu *.Mask))
  (pad 5 thru_hole oval (at 0 2.54) (size 1.7 1.7) (drill 1) (layers *.Cu *.Mask))
  (pad 6 thru_hole oval (at -2.54 2.54) (size 1.7 1.7) (drill 1) (layers *.Cu *.Mask))
  (pad 9 thru_hole oval (at 0 5.08) (size 1.7 1.7) (drill 1) (layers *.Cu *.Mask))
  (pad 10 thru_hole oval (at -2.54 5.08) (size 1.7 1.7) (drill 1) (layers *.Cu *.Mask))
  (pad 3 thru_hole oval (at -5.08 0) (size 1.7 1.7) (drill 1) (layers *.Cu *.Mask))
  (pad 7 thru_hole oval (at -5.08 2.54) (size 1.7 1.7) (drill 1) (layers *.Cu *.Mask))
  (pad 11 thru_hole oval (at -5.08 5.08) (size 1.7 1.7) (drill 1) (layers *.Cu *.Mask)))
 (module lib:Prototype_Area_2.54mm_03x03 (layer F.Cu) (at 156.21 88.9)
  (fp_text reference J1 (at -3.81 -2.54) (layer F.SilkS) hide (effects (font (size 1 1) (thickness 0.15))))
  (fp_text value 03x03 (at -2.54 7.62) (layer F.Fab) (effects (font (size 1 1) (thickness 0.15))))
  (fp_line (start -6.35 6.35) (end -6.35 -1.27) (layer F.SilkS) (width 0.15))
  (fp_line (start 1.27 6.35) (end -6.35 6.35) (layer F.SilkS) (width 0.15))
  (fp_line (start 1.27 -1.27) (end 1.27 6.35) (layer F.SilkS) (width 0.15))
  (fp_line (start -6.35 -1.27) (end 1.27 -1.27) (layer F.SilkS) (width 0.15))
  (pad 1 thru_hole circle (at 0 0) (size 1.7 1.7) (drill 1) (layers *.Cu *.Mask))
  (pad 2 thru_hole oval (at -2.54 0) (size 1.7 1.7) (drill 1) (layers *.Cu *.Mask))
  (pad 5 thru_hole oval (at 0 2.54) (size 1.7 1.7) (drill 1) (layers *.Cu *.Mask))
  (pad 6 thru_hole oval (at -2.54 2.54) (size 1.7 1.7) (drill 1) (layers *.Cu *.Mask))
  (pad 9 thru_hole oval (at 0 5.08) (size 1.7 1.7) (drill 1) (layers *.Cu *.Mask))
  (pad 10 thru_hole oval (at -2.54 5.08) (size 1.7 1.7) (drill 1) (layers *.Cu *.Mask))
  (pad 3 thru_hole oval (at -5.08 0) (size 1.7 1.7) (drill 1) (layers *.Cu *.Mask))
  (pad 7 thru_hole oval (at -5.08 2.54) (size 1.7 1.7) (drill 1) (layers *.Cu *.Mask))
  (pad 11 thru_hole oval (at -5.08 5.08) (size 1.7 1.7) (drill 1) (layers *.Cu *.Mask)))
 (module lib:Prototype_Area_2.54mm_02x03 (layer F.Cu) (at 151.13 109.22 90)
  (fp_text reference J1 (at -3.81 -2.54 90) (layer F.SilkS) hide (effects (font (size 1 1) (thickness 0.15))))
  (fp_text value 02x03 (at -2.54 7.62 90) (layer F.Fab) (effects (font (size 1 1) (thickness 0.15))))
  (fp_line (start -3.81 6.35) (end -3.81 -1.27) (layer F.SilkS) (width 0.15))
  (fp_line (start 1.27 6.35) (end -3.81 6.35) (layer F.SilkS) (width 0.15))
  (fp_line (start 1.27 -1.27) (end 1.27 6.35) (layer F.SilkS) (width 0.15))
  (fp_line (start -3.81 -1.27) (end 1.27 -1.27) (layer F.SilkS) (width 0.15))
  (pad 1 thru_hole circle (at 0 0 90) (size 1.7 1.7) (drill 1) (layers *.Cu *.Mask))
  (pad 2 thru_hole oval (at -2.54 0 90) (size 1.7 1.7) (drill 1) (layers *.Cu *.Mask))
  (pad 3 thru_hole oval (at 0 2.54 90) (size 1.7 1.7) (drill 1) (layers *.Cu *.Mask))
  (pad 4 thru_hole oval (at -2.54 2.54 90) (size 1.7 1.7) (drill 1) (layers *.Cu *.Mask))
  (pad 5 thru_hole oval (at 0 5.08 90) (size 1.7 1.7) (drill 1) (layers *.Cu *.Mask))
  (pad 6 thru_hole oval (at -2.54 5.08 90) (size 1.7 1.7) (drill 1) (layers *.Cu *.Mask)))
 (gr_arc (start 143.51 111.76) (end 140.97 111.76) (angle -90) (layer Edge.Cuts) (width 0.15))
 (gr_arc (start 143.51 88.9) (end 143.51 86.36) (angle -90) (layer Edge.Cuts) (width 0.15))
 (gr_arc (start 191.77 111.76) (end 191.77 114.3) (angle -90) (layer Edge.Cuts) (width 0.15))
 (gr_arc (start 191.77 88.9) (end 194.31 88.9) (angle -90) (layer Edge.Cuts) (width 0.15))
 (gr_line (start 140.97 111.76) (end 140.97 88.9) (layer Edge.Cuts) (width 0.15))
 (gr_line (start 191.77 114.3) (end 143.51 114.3) (layer Edge.Cuts) (width 0.15))
 (gr_line (start 194.31 88.9) (end 194.31 111.76) (layer Edge.Cuts) (width 0.15))
 (gr_line (start 143.51 86.36) (end 191.77 86.36) (layer Edge.Cuts) (width 0.15))
 (via (at 193.167 97.79) (size 2) (drill 1) (layers F.Cu B.Cu) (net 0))
 (via (at 193.167 102.87) (size 2) (drill 1) (layers F.Cu B.Cu) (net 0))
 (via (at 142.24 97.79) (size 2) (drill 1) (layers F.Cu B.Cu) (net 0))
 (via (at 142.24 102.87) (size 2) (drill 1) (layers F.Cu B.Cu) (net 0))
 (segment (start 185.928 96.52) (end 187.198 97.79) (width 1) (layer F.Cu) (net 1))
 (segment (start 184.15 96.52) (end 185.928 96.52) (width 1) (layer F.Cu) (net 1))
 (segment (start 187.198 100.076) (end 188.722 101.6) (width 1) (layer F.Cu) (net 1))
 (segment (start 187.198 97.79) (end 187.198 100.076) (width 1) (layer F.Cu) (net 1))
 (segment (start 146.685 101.981) (end 148.082 103.378) (width 1) (layer F.Cu) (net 4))
 (segment (start 146.685 99.314) (end 146.685 101.981) (width 1) (layer F.Cu) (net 4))
 (segment (start 150.114 103.378) (end 151.257 104.521) (width 1) (layer F.Cu) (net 4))
 (segment (start 148.082 103.378) (end 150.114 103.378) (width 1) (layer F.Cu) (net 4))
 (segment (start 188.92 95.29) (end 190.15 96.52) (width 1) (layer F.Cu) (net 2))
 (segment (start 187.198 95.29) (end 188.92 95.29) (width 1) (layer F.Cu) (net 2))
 (segment (start 187.15 95.242) (end 187.198 95.29) (width 1) (layer F.Cu) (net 2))
 (segment (start 187.15 91.82) (end 187.15 95.242) (width 1) (layer F.Cu) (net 2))
 (segment (start 190.221999 105.180001) (end 188.722 106.68) (width 1) (layer F.Cu) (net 2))
 (segment (start 190.922001 104.479999) (end 190.221999 105.180001) (width 1) (layer F.Cu) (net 2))
 (segment (start 190.922001 99.142001) (end 190.922001 104.479999) (width 1) (layer F.Cu) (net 2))
 (segment (start 190.15 98.37) (end 190.922001 99.142001) (width 1) (layer F.Cu) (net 2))
 (segment (start 190.15 96.52) (end 190.15 98.37) (width 1) (layer F.Cu) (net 2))
 (segment (start 145.257 102.671) (end 145.257 104.521) (width 1) (layer F.Cu) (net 3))
 (segment (start 143.940001 101.354001) (end 145.257 102.671) (width 1) (layer F.Cu) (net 3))
 (segment (start 143.940001 96.978999) (end 143.940001 101.354001) (width 1) (layer F.Cu) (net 3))
 (segment (start 146.685 94.234) (end 143.940001 96.978999) (width 1) (layer F.Cu) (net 3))
 (segment (start 146.614 105.878) (end 148.082 105.878) (width 1) (layer F.Cu) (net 3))
 (segment (start 145.257 104.521) (end 146.614 105.878) (width 1) (layer F.Cu) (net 3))
 (segment (start 148.082 109.046) (end 148.257 109.221) (width 1) (layer F.Cu) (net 3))
 (segment (start 148.082 105.878) (end 148.082 109.046) (width 1) (layer F.Cu) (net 3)))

